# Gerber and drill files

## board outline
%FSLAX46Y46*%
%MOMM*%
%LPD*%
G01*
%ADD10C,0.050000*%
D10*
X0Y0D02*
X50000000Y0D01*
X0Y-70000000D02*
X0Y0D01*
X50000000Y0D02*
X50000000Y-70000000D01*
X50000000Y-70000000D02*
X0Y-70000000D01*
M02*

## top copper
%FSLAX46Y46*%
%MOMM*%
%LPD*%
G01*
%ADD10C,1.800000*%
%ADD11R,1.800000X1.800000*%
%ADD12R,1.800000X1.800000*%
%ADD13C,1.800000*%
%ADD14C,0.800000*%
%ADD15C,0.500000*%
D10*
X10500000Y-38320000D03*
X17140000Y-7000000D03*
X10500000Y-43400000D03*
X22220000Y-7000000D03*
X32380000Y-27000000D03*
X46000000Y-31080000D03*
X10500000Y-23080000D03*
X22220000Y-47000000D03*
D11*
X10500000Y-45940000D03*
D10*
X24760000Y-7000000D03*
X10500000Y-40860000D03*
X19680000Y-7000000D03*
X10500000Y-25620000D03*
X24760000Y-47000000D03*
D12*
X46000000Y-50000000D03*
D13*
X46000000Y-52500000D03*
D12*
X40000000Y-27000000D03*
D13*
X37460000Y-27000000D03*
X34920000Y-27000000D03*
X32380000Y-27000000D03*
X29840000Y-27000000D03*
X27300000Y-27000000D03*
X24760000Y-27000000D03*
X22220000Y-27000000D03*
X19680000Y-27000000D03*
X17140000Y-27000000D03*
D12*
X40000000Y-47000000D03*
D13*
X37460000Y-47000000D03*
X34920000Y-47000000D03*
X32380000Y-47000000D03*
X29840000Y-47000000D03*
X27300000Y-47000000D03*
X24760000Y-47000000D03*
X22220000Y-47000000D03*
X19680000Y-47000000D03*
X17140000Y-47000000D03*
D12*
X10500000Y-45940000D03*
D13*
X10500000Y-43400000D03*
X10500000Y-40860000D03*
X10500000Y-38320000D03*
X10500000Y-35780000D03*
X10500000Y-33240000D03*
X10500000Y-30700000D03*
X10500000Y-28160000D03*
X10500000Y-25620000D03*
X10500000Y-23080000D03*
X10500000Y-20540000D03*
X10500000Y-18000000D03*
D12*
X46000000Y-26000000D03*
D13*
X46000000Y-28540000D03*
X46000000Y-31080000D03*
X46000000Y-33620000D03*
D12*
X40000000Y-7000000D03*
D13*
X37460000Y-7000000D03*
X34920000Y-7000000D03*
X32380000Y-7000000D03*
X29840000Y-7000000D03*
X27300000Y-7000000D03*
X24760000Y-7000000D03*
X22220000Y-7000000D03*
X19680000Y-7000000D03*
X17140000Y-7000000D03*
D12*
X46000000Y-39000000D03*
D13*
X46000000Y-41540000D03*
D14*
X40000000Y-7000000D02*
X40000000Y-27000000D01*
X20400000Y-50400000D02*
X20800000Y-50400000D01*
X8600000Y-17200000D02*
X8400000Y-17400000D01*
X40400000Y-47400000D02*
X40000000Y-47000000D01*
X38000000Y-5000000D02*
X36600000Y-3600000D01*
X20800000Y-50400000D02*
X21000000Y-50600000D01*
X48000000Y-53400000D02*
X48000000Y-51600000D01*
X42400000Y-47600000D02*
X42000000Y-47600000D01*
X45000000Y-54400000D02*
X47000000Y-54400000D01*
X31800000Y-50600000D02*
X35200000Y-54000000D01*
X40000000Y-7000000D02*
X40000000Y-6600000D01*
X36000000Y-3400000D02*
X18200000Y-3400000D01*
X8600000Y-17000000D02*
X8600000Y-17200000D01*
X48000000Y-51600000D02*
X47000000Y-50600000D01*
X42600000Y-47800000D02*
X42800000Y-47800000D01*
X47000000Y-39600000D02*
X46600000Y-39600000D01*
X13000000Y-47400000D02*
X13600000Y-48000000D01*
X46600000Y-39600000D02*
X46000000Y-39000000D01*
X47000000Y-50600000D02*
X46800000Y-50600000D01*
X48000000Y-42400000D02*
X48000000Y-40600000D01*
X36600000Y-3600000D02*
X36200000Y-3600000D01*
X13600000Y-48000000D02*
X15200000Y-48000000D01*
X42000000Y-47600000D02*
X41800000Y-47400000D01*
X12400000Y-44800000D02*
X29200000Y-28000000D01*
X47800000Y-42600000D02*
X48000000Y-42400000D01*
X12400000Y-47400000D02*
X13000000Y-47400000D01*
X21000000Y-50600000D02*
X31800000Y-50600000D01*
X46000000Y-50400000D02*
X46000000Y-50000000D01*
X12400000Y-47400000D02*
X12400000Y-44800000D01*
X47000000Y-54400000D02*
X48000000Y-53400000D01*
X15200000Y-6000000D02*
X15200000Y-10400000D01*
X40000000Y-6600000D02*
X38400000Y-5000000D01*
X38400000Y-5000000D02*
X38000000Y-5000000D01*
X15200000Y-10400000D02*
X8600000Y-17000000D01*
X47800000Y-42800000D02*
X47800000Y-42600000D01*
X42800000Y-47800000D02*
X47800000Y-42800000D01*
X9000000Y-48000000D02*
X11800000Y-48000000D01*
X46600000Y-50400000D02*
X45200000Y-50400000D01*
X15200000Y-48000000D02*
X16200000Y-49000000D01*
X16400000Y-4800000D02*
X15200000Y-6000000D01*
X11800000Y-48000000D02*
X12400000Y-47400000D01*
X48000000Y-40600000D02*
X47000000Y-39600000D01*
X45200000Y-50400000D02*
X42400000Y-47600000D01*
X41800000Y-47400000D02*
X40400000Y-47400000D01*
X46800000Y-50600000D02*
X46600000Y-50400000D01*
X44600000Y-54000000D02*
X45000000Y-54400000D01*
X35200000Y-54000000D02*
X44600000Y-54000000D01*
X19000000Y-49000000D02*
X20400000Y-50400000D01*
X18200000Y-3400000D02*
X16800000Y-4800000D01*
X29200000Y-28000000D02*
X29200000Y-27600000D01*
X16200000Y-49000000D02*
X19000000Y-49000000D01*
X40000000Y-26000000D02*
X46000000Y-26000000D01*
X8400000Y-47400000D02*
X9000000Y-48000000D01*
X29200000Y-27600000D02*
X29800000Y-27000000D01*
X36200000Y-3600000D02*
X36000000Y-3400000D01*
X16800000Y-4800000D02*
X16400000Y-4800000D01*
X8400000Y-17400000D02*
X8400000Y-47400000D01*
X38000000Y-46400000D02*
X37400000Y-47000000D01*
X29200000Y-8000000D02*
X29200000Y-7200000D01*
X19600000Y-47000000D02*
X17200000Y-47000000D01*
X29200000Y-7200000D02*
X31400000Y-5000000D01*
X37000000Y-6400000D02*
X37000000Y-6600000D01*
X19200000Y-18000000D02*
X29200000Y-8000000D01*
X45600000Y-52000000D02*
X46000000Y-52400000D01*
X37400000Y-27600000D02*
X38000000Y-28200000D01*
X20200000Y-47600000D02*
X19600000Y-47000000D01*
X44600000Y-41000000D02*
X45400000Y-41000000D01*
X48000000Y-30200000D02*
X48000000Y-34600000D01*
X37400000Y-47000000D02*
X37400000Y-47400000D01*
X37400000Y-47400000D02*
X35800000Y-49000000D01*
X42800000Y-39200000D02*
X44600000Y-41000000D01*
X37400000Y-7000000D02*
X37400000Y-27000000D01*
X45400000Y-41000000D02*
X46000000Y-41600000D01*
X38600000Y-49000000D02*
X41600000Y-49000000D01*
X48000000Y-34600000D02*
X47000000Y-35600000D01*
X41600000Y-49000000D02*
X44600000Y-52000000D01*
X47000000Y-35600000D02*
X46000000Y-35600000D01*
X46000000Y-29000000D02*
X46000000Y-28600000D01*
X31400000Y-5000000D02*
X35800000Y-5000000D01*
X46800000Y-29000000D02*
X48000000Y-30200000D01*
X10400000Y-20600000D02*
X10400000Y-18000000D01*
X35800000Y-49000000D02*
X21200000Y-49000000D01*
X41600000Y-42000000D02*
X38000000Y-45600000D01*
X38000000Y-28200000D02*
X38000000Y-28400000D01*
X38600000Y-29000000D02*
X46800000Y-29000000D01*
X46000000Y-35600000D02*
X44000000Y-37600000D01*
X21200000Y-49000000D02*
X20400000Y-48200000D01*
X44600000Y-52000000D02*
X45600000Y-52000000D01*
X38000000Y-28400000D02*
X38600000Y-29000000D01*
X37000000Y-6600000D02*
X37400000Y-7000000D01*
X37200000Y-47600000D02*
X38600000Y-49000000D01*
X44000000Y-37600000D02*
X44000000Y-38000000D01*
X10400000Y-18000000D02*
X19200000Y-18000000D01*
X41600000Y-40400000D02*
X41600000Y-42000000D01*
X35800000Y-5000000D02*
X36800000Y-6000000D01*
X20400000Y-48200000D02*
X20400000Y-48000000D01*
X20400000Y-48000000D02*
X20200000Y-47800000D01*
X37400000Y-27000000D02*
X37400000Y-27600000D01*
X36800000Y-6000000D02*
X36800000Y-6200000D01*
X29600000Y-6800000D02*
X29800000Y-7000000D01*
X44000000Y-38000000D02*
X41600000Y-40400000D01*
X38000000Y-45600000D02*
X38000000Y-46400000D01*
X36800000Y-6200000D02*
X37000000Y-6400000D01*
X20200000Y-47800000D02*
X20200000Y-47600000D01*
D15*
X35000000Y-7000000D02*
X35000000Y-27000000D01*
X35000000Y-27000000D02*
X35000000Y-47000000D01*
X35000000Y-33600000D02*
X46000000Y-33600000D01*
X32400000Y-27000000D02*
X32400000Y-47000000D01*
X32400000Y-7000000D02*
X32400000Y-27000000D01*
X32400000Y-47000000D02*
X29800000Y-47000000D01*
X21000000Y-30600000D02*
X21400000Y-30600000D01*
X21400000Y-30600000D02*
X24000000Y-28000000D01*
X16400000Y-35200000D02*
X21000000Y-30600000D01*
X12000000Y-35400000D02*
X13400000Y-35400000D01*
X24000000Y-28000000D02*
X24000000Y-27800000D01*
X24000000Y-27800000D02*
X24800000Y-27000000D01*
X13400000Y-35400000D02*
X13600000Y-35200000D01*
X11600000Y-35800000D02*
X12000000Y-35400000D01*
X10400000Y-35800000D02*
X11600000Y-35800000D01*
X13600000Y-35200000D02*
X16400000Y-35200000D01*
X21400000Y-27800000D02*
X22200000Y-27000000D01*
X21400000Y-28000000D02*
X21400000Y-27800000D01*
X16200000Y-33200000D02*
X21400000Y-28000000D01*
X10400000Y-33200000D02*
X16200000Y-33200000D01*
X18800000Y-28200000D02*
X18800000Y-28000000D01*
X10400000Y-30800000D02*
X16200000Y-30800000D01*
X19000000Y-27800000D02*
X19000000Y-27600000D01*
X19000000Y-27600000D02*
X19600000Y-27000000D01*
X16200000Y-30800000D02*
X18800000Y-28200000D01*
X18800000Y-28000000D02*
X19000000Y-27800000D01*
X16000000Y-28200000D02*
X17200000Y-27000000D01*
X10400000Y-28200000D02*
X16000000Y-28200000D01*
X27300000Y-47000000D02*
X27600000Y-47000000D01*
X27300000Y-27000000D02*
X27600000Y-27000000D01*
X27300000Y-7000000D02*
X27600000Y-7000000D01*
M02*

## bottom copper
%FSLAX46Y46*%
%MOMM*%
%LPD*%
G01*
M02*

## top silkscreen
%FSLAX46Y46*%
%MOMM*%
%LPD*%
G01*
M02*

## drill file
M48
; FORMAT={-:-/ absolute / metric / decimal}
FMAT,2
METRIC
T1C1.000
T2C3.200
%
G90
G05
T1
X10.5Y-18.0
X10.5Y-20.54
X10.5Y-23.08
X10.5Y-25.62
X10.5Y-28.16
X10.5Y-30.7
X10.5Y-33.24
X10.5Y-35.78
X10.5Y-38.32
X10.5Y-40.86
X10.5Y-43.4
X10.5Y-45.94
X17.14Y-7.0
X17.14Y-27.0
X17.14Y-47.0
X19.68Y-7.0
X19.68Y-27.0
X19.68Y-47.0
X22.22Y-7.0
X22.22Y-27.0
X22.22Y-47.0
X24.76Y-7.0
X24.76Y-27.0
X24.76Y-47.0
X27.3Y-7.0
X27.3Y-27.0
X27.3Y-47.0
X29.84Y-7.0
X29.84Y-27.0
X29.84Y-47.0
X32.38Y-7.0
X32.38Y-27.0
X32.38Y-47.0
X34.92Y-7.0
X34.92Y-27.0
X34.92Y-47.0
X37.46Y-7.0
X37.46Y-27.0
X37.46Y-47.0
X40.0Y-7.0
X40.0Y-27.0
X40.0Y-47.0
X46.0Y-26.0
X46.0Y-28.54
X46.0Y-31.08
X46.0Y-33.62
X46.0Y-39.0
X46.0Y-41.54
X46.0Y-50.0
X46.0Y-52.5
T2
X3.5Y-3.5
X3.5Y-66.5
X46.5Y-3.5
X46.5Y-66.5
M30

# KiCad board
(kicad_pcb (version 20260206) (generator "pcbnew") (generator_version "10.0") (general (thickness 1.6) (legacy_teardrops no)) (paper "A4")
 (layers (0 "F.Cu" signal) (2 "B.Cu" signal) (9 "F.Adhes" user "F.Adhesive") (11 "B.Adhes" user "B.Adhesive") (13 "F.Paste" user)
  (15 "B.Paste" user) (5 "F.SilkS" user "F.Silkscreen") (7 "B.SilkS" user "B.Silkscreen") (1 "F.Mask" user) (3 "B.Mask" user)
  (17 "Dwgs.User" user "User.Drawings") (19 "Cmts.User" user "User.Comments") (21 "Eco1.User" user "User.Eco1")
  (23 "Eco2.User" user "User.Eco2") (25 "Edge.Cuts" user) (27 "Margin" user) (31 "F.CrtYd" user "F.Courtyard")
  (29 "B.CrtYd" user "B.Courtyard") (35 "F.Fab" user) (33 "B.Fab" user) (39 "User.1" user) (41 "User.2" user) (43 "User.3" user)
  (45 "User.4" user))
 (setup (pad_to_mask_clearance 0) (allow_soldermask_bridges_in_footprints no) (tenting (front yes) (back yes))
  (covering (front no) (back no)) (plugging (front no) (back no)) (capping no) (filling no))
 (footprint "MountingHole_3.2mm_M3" (layer "F.Cu") (at 3.5 3.5)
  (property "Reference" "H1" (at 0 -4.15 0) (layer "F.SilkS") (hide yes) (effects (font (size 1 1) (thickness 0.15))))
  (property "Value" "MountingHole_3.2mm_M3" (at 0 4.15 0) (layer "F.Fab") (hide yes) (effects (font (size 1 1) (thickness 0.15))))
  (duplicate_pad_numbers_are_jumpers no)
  (pad "" np_thru_hole circle (at 0 0) (size 3.2 3.2) (drill 3.2) (layers "*.Cu" "*.Mask")))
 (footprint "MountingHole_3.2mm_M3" (layer "F.Cu") (at 46.5 66.5)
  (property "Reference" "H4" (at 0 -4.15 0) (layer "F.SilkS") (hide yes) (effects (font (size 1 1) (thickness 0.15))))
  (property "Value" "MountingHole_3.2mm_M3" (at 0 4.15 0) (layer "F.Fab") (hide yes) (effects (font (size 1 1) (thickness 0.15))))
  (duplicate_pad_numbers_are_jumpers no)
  (pad "" np_thru_hole circle (at 0 0) (size 3.2 3.2) (drill 3.2) (layers "*.Cu" "*.Mask")))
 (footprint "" (layer "F.Cu") (at 0 0)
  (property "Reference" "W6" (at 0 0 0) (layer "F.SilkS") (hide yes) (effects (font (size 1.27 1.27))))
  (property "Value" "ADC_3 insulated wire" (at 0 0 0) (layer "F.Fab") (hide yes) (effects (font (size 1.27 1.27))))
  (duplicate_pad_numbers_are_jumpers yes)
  (pad "1" smd circle (at 10.5 38.32) (size 1.8 1.8) (layers "F.Cu") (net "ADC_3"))
  (pad "1" smd circle (at 17.14 7) (size 1.8 1.8) (layers "F.Cu") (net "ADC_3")))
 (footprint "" (layer "F.Cu") (at 0 0)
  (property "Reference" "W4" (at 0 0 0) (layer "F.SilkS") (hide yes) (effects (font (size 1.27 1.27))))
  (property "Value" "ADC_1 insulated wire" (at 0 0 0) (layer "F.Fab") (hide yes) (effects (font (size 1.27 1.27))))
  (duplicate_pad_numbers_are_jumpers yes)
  (pad "1" smd circle (at 10.5 43.4) (size 1.8 1.8) (layers "F.Cu") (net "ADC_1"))
  (pad "1" smd circle (at 22.22 7) (size 1.8 1.8) (layers "F.Cu") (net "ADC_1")))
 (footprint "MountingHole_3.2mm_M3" (layer "F.Cu") (at 3.5 66.5)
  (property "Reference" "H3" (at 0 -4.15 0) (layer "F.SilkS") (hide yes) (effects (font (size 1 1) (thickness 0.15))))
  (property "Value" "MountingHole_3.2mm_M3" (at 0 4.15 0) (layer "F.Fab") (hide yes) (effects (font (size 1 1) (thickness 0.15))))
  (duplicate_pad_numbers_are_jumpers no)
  (pad "" np_thru_hole circle (at 0 0) (size 3.2 3.2) (drill 3.2) (layers "*.Cu" "*.Mask")))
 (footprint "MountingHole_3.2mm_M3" (layer "F.Cu") (at 46.5 3.5)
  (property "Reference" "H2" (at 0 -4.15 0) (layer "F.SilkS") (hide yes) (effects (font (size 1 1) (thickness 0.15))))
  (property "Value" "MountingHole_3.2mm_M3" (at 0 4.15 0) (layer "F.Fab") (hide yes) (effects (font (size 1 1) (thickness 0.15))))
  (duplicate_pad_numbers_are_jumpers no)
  (pad "" np_thru_hole circle (at 0 0) (size 3.2 3.2) (drill 3.2) (layers "*.Cu" "*.Mask")))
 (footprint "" (layer "F.Cu") (at 0 0)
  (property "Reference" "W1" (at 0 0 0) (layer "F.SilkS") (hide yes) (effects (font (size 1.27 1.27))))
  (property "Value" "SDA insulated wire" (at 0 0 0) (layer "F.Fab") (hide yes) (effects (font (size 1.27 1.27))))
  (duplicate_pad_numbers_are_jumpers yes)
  (pad "1" smd circle (at 32.38 27) (size 1.8 1.8) (layers "F.Cu") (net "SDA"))
  (pad "1" smd circle (at 46 31.08) (size 1.8 1.8) (layers "F.Cu") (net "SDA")))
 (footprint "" (layer "F.Cu") (at 0 0)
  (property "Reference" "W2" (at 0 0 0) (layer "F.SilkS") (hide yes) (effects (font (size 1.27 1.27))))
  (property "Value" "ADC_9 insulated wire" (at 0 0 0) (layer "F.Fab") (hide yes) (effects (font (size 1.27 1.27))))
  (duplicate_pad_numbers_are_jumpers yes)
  (pad "1" smd circle (at 10.5 23.08) (size 1.8 1.8) (layers "F.Cu") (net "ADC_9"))
  (pad "1" smd circle (at 22.22 47) (size 1.8 1.8) (layers "F.Cu") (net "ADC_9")))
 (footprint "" (layer "F.Cu") (at 0 0)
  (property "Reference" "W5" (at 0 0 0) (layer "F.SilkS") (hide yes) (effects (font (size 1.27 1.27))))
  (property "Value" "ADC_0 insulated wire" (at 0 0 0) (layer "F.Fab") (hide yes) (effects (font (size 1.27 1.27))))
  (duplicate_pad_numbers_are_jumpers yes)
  (pad "1" smd rect (at 10.5 45.94) (size 1.8 1.8) (layers "F.Cu") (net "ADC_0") (thermal_bridge_angle 45))
  (pad "1" smd circle (at 24.76 7) (size 1.8 1.8) (layers "F.Cu") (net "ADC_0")))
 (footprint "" (layer "F.Cu") (at 0 0)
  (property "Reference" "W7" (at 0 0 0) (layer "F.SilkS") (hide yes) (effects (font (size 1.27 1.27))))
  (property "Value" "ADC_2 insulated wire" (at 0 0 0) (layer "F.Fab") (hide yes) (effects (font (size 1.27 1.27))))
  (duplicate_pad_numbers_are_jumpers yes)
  (pad "1" smd circle (at 10.5 40.86) (size 1.8 1.8) (layers "F.Cu") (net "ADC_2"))
  (pad "1" smd circle (at 19.68 7) (size 1.8 1.8) (layers "F.Cu") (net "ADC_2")))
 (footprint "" (layer "F.Cu") (at 0 0)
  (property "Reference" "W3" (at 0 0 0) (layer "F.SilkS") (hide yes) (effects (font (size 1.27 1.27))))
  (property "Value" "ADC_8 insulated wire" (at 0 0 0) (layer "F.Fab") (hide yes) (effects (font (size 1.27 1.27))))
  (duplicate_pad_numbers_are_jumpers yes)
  (pad "1" smd circle (at 10.5 25.62) (size 1.8 1.8) (layers "F.Cu") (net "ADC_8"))
  (pad "1" smd circle (at 24.76 47) (size 1.8 1.8) (layers "F.Cu") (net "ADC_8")))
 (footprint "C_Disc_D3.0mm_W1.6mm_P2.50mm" (layer "B.Cu") (at 46 50 -90)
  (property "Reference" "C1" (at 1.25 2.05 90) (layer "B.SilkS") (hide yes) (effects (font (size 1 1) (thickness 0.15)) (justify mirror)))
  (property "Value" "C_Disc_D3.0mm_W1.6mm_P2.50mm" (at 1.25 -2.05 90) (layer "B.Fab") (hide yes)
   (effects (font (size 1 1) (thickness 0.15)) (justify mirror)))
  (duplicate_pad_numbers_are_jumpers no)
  (pad "1" thru_hole rect (at 0 0 270) (size 1.8 1.8) (drill 1) (layers "*.Mask" "F.Cu") (remove_unused_layers yes) (keep_end_layers no)
   (zone_layer_connections) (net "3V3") (thermal_bridge_angle 45))
  (pad "2" thru_hole circle (at 2.5 0 270) (size 1.8 1.8) (drill 1) (layers "*.Mask" "F.Cu") (remove_unused_layers yes) (keep_end_layers no)
   (zone_layer_connections) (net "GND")))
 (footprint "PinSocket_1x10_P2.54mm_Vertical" (layer "B.Cu") (at 40 27 90)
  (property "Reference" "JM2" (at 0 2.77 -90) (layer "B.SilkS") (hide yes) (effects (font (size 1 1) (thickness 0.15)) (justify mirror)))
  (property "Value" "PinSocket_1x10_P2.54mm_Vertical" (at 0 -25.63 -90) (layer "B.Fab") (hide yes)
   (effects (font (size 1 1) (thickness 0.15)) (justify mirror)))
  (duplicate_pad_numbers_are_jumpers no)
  (pad "1" thru_hole rect (at 0 0 90) (size 1.8 1.8) (drill 1) (layers "*.Mask" "F.Cu") (remove_unused_layers yes) (keep_end_layers no)
   (zone_layer_connections) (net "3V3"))
  (pad "2" thru_hole circle (at 0 -2.54 90) (size 1.8 1.8) (drill 1) (layers "*.Mask" "F.Cu") (remove_unused_layers yes)
   (keep_end_layers no) (zone_layer_connections) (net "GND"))
  (pad "3" thru_hole circle (at 0 -5.08 90) (size 1.8 1.8) (drill 1) (layers "*.Mask" "F.Cu") (remove_unused_layers yes)
   (keep_end_layers no) (zone_layer_connections) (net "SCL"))
  (pad "4" thru_hole circle (at 0 -7.62 90) (size 1.8 1.8) (drill 1) (layers "*.Mask" "F.Cu") (remove_unused_layers yes)
   (keep_end_layers no) (zone_layer_connections) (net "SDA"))
  (pad "5" thru_hole circle (at 0 -10.16 90) (size 1.8 1.8) (drill 1) (layers "*.Mask" "F.Cu") (remove_unused_layers yes)
   (keep_end_layers no) (zone_layer_connections) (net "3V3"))
  (pad "6" thru_hole circle (at 0 -12.7 90) (size 1.8 1.8) (drill 1) (layers "*.Mask" "F.Cu") (remove_unused_layers yes)
   (keep_end_layers no) (zone_layer_connections) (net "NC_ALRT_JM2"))
  (pad "7" thru_hole circle (at 0 -15.24 90) (size 1.8 1.8) (drill 1) (layers "*.Mask" "F.Cu") (remove_unused_layers yes)
   (keep_end_layers no) (zone_layer_connections) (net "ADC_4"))
  (pad "8" thru_hole circle (at 0 -17.78 90) (size 1.8 1.8) (drill 1) (layers "*.Mask" "F.Cu") (remove_unused_layers yes)
   (keep_end_layers no) (zone_layer_connections) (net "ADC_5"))
  (pad "9" thru_hole circle (at 0 -20.32 90) (size 1.8 1.8) (drill 1) (layers "*.Mask" "F.Cu") (remove_unused_layers yes)
   (keep_end_layers no) (zone_layer_connections) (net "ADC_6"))
  (pad "10" thru_hole circle (at 0 -22.86 90) (size 1.8 1.8) (drill 1) (layers "*.Mask" "F.Cu") (remove_unused_layers yes)
   (keep_end_layers no) (zone_layer_connections) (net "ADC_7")))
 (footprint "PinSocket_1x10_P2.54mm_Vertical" (layer "B.Cu") (at 40 47 90)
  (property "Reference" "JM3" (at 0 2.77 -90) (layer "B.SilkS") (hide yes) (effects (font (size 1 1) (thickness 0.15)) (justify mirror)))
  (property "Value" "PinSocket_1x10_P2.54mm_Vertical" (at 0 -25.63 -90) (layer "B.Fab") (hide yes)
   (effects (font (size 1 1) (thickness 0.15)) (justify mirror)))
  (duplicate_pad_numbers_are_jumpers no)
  (pad "1" thru_hole rect (at 0 0 90) (size 1.8 1.8) (drill 1) (layers "*.Mask" "F.Cu") (remove_unused_layers yes) (keep_end_layers no)
   (zone_layer_connections) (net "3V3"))
  (pad "2" thru_hole circle (at 0 -2.54 90) (size 1.8 1.8) (drill 1) (layers "*.Mask" "F.Cu") (remove_unused_layers yes)
   (keep_end_layers no) (zone_layer_connections) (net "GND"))
  (pad "3" thru_hole circle (at 0 -5.08 90) (size 1.8 1.8) (drill 1) (layers "*.Mask" "F.Cu") (remove_unused_layers yes)
   (keep_end_layers no) (zone_layer_connections) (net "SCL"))
  (pad "4" thru_hole circle (at 0 -7.62 90) (size 1.8 1.8) (drill 1) (layers "*.Mask" "F.Cu") (remove_unused_layers yes)
   (keep_end_layers no) (zone_layer_connections) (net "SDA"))
  (pad "5" thru_hole circle (at 0 -10.16 90) (size 1.8 1.8) (drill 1) (layers "*.Mask" "F.Cu") (remove_unused_layers yes)
   (keep_end_layers no) (zone_layer_connections) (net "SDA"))
  (pad "6" thru_hole circle (at 0 -12.7 90) (size 1.8 1.8) (drill 1) (layers "*.Mask" "F.Cu") (remove_unused_layers yes)
   (keep_end_layers no) (zone_layer_connections) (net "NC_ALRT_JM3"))
  (pad "7" thru_hole circle (at 0 -15.24 90) (size 1.8 1.8) (drill 1) (layers "*.Mask" "F.Cu") (remove_unused_layers yes)
   (keep_end_layers no) (zone_layer_connections) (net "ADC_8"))
  (pad "8" thru_hole circle (at 0 -17.78 90) (size 1.8 1.8) (drill 1) (layers "*.Mask" "F.Cu") (remove_unused_layers yes)
   (keep_end_layers no) (zone_layer_connections) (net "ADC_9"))
  (pad "9" thru_hole circle (at 0 -20.32 90) (size 1.8 1.8) (drill 1) (layers "*.Mask" "F.Cu") (remove_unused_layers yes)
   (keep_end_layers no) (zone_layer_connections) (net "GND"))
  (pad "10" thru_hole circle (at 0 -22.86 90) (size 1.8 1.8) (drill 1) (layers "*.Mask" "F.Cu") (remove_unused_layers yes)
   (keep_end_layers no) (zone_layer_connections) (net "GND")))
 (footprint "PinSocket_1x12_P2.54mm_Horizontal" (layer "B.Cu") (at 10.5 45.94)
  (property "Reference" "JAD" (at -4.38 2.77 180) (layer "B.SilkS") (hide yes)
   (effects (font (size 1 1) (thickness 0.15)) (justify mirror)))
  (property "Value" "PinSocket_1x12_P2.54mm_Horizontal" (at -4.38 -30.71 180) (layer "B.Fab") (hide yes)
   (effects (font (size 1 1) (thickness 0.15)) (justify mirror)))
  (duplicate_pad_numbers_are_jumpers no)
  (pad "1" thru_hole rect (at 0 0) (size 1.8 1.8) (drill 1) (layers "*.Mask" "F.Cu") (remove_unused_layers yes) (keep_end_layers no)
   (zone_layer_connections) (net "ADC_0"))
  (pad "2" thru_hole circle (at 0 -2.54) (size 1.8 1.8) (drill 1) (layers "*.Mask" "F.Cu") (remove_unused_layers yes) (keep_end_layers no)
   (zone_layer_connections) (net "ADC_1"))
  (pad "3" thru_hole circle (at 0 -5.08) (size 1.8 1.8) (drill 1) (layers "*.Mask" "F.Cu") (remove_unused_layers yes) (keep_end_layers no)
   (zone_layer_connections) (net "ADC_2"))
  (pad "4" thru_hole circle (at 0 -7.62) (size 1.8 1.8) (drill 1) (layers "*.Mask" "F.Cu") (remove_unused_layers yes) (keep_end_layers no)
   (zone_layer_connections) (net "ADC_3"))
  (pad "5" thru_hole circle (at 0 -10.16) (size 1.8 1.8) (drill 1) (layers "*.Mask" "F.Cu") (remove_unused_layers yes) (keep_end_layers no)
   (zone_layer_connections) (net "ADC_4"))
  (pad "6" thru_hole circle (at 0 -12.7) (size 1.8 1.8) (drill 1) (layers "*.Mask" "F.Cu") (remove_unused_layers yes) (keep_end_layers no)
   (zone_layer_connections) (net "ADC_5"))
  (pad "7" thru_hole circle (at 0 -15.24) (size 1.8 1.8) (drill 1) (layers "*.Mask" "F.Cu") (remove_unused_layers yes) (keep_end_layers no)
   (zone_layer_connections) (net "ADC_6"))
  (pad "8" thru_hole circle (at 0 -17.78) (size 1.8 1.8) (drill 1) (layers "*.Mask" "F.Cu") (remove_unused_layers yes) (keep_end_layers no)
   (zone_layer_connections) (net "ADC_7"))
  (pad "9" thru_hole circle (at 0 -20.32) (size 1.8 1.8) (drill 1) (layers "*.Mask" "F.Cu") (remove_unused_layers yes) (keep_end_layers no)
   (zone_layer_connections) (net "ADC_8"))
  (pad "10" thru_hole circle (at 0 -22.86) (size 1.8 1.8) (drill 1) (layers "*.Mask" "F.Cu") (remove_unused_layers yes) (keep_end_layers no)
   (zone_layer_connections) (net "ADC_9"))
  (pad "11" thru_hole circle (at 0 -25.4) (size 1.8 1.8) (drill 1) (layers "*.Mask" "F.Cu") (remove_unused_layers yes) (keep_end_layers no)
   (zone_layer_connections) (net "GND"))
  (pad "12" thru_hole circle (at 0 -27.94) (size 1.8 1.8) (drill 1) (layers "*.Mask" "F.Cu") (remove_unused_layers yes) (keep_end_layers no)
   (zone_layer_connections) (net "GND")))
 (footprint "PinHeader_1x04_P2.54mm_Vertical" (layer "B.Cu") (at 46 26 180)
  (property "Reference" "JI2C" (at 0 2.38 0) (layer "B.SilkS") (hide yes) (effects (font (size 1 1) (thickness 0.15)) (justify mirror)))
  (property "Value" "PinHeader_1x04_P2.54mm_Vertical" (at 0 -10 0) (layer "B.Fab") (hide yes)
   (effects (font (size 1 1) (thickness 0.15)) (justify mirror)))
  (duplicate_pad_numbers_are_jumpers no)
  (pad "1" thru_hole rect (at 0 0 180) (size 1.8 1.8) (drill 1) (layers "*.Mask" "F.Cu") (remove_unused_layers yes) (keep_end_layers no)
   (zone_layer_connections) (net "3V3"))
  (pad "2" thru_hole circle (at 0 -2.54 180) (size 1.8 1.8) (drill 1) (layers "*.Mask" "F.Cu") (remove_unused_layers yes)
   (keep_end_layers no) (zone_layer_connections) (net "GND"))
  (pad "3" thru_hole circle (at 0 -5.08 180) (size 1.8 1.8) (drill 1) (layers "*.Mask" "F.Cu") (remove_unused_layers yes)
   (keep_end_layers no) (zone_layer_connections) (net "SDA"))
  (pad "4" thru_hole circle (at 0 -7.62 180) (size 1.8 1.8) (drill 1) (layers "*.Mask" "F.Cu") (remove_unused_layers yes)
   (keep_end_layers no) (zone_layer_connections) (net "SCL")))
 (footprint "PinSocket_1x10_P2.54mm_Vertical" (layer "B.Cu") (at 40 7 90)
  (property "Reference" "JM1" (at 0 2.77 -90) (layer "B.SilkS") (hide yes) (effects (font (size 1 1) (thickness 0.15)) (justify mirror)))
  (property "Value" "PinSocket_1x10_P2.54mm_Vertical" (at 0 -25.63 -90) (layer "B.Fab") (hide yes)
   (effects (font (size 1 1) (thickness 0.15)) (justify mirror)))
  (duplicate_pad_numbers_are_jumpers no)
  (pad "1" thru_hole rect (at 0 0 90) (size 1.8 1.8) (drill 1) (layers "*.Mask" "F.Cu") (remove_unused_layers yes) (keep_end_layers no)
   (zone_layer_connections) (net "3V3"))
  (pad "2" thru_hole circle (at 0 -2.54 90) (size 1.8 1.8) (drill 1) (layers "*.Mask" "F.Cu") (remove_unused_layers yes)
   (keep_end_layers no) (zone_layer_connections) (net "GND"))
  (pad "3" thru_hole circle (at 0 -5.08 90) (size 1.8 1.8) (drill 1) (layers "*.Mask" "F.Cu") (remove_unused_layers yes)
   (keep_end_layers no) (zone_layer_connections) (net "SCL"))
  (pad "4" thru_hole circle (at 0 -7.62 90) (size 1.8 1.8) (drill 1) (layers "*.Mask" "F.Cu") (remove_unused_layers yes)
   (keep_end_layers no) (zone_layer_connections) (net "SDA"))
  (pad "5" thru_hole circle (at 0 -10.16 90) (size 1.8 1.8) (drill 1) (layers "*.Mask" "F.Cu") (remove_unused_layers yes)
   (keep_end_layers no) (zone_layer_connections) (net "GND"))
  (pad "6" thru_hole circle (at 0 -12.7 90) (size 1.8 1.8) (drill 1) (layers "*.Mask" "F.Cu") (remove_unused_layers yes)
   (keep_end_layers no) (zone_layer_connections) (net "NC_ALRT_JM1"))
  (pad "7" thru_hole circle (at 0 -15.24 90) (size 1.8 1.8) (drill 1) (layers "*.Mask" "F.Cu") (remove_unused_layers yes)
   (keep_end_layers no) (zone_layer_connections) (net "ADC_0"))
  (pad "8" thru_hole circle (at 0 -17.78 90) (size 1.8 1.8) (drill 1) (layers "*.Mask" "F.Cu") (remove_unused_layers yes)
   (keep_end_layers no) (zone_layer_connections) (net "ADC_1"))
  (pad "9" thru_hole circle (at 0 -20.32 90) (size 1.8 1.8) (drill 1) (layers "*.Mask" "F.Cu") (remove_unused_layers yes)
   (keep_end_layers no) (zone_layer_connections) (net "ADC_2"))
  (pad "10" thru_hole circle (at 0 -22.86 90) (size 1.8 1.8) (drill 1) (layers "*.Mask" "F.Cu") (remove_unused_layers yes)
   (keep_end_layers no) (zone_layer_connections) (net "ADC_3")))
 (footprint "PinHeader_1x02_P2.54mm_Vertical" (layer "B.Cu") (at 46 39 180)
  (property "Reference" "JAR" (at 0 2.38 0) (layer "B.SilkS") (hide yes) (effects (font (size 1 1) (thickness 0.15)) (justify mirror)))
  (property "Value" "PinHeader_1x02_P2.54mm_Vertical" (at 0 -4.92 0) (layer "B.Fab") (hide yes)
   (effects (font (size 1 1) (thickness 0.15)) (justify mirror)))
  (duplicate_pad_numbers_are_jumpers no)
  (pad "1" thru_hole rect (at 0 0 180) (size 1.8 1.8) (drill 1) (layers "*.Mask" "F.Cu") (remove_unused_layers yes) (keep_end_layers no)
   (zone_layer_connections) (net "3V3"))
  (pad "2" thru_hole circle (at 0 -2.54 180) (size 1.8 1.8) (drill 1) (layers "*.Mask" "F.Cu") (remove_unused_layers yes)
   (keep_end_layers no) (zone_layer_connections) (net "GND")))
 (gr_line (start 0 0) (end 50 0) (stroke (width 0.05) (type default)) (layer "Edge.Cuts"))
 (gr_line (start 0 70) (end 0 0) (stroke (width 0.05) (type default)) (layer "Edge.Cuts"))
 (gr_line (start 50 0) (end 50 70) (stroke (width 0.05) (type default)) (layer "Edge.Cuts"))
 (gr_line (start 50 70) (end 0 70) (stroke (width 0.05) (type default)) (layer "Edge.Cuts"))
 (segment (start 40 7) (end 40 27) (width 0.8) (layer "F.Cu") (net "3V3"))
 (segment (start 20.4 50.4) (end 20.8 50.4) (width 0.8) (layer "F.Cu") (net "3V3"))
 (segment (start 8.6 17.2) (end 8.4 17.4) (width 0.8) (layer "F.Cu") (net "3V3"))
 (segment (start 40.4 47.4) (end 40 47) (width 0.8) (layer "F.Cu") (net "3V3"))
 (segment (start 38 5) (end 36.6 3.6) (width 0.8) (layer "F.Cu") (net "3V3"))
 (segment (start 20.8 50.4) (end 21 50.6) (width 0.8) (layer "F.Cu") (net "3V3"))
 (segment (start 48 53.4) (end 48 51.6) (width 0.8) (layer "F.Cu") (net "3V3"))
 (segment (start 42.4 47.6) (end 42 47.6) (width 0.8) (layer "F.Cu") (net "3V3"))
 (segment (start 45 54.4) (end 47 54.4) (width 0.8) (layer "F.Cu") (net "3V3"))
 (segment (start 31.8 50.6) (end 35.2 54) (width 0.8) (layer "F.Cu") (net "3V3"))
 (segment (start 40 7) (end 40 6.6) (width 0.8) (layer "F.Cu") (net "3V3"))
 (segment (start 36 3.4) (end 18.2 3.4) (width 0.8) (layer "F.Cu") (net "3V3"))
 (segment (start 8.6 17) (end 8.6 17.2) (width 0.8) (layer "F.Cu") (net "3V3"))
 (segment (start 48 51.6) (end 47 50.6) (width 0.8) (layer "F.Cu") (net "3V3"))
 (segment (start 42.6 47.8) (end 42.8 47.8) (width 0.8) (layer "F.Cu") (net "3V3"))
 (segment (start 47 39.6) (end 46.6 39.6) (width 0.8) (layer "F.Cu") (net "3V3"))
 (segment (start 13 47.4) (end 13.6 48) (width 0.8) (layer "F.Cu") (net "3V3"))
 (segment (start 46.6 39.6) (end 46 39) (width 0.8) (layer "F.Cu") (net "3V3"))
 (segment (start 47 50.6) (end 46.8 50.6) (width 0.8) (layer "F.Cu") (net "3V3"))
 (segment (start 48 42.4) (end 48 40.6) (width 0.8) (layer "F.Cu") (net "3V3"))
 (segment (start 36.6 3.6) (end 36.2 3.6) (width 0.8) (layer "F.Cu") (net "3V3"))
 (segment (start 13.6 48) (end 15.2 48) (width 0.8) (layer "F.Cu") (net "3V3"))
 (segment (start 42 47.6) (end 41.8 47.4) (width 0.8) (layer "F.Cu") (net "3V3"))
 (segment (start 12.4 44.8) (end 29.2 28) (width 0.8) (layer "F.Cu") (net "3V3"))
 (segment (start 47.8 42.6) (end 48 42.4) (width 0.8) (layer "F.Cu") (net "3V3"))
 (segment (start 12.4 47.4) (end 13 47.4) (width 0.8) (layer "F.Cu") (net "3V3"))
 (segment (start 21 50.6) (end 31.8 50.6) (width 0.8) (layer "F.Cu") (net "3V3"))
 (segment (start 46 50.4) (end 46 50) (width 0.8) (layer "F.Cu") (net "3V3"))
 (segment (start 12.4 47.4) (end 12.4 44.8) (width 0.8) (layer "F.Cu") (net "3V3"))
 (segment (start 47 54.4) (end 48 53.4) (width 0.8) (layer "F.Cu") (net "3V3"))
 (segment (start 15.2 6) (end 15.2 10.4) (width 0.8) (layer "F.Cu") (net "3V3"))
 (segment (start 40 6.6) (end 38.4 5) (width 0.8) (layer "F.Cu") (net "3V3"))
 (segment (start 38.4 5) (end 38 5) (width 0.8) (layer "F.Cu") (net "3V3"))
 (segment (start 15.2 10.4) (end 8.6 17) (width 0.8) (layer "F.Cu") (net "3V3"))
 (segment (start 47.8 42.8) (end 47.8 42.6) (width 0.8) (layer "F.Cu") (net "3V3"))
 (segment (start 42.8 47.8) (end 47.8 42.8) (width 0.8) (layer "F.Cu") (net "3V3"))
 (segment (start 9 48) (end 11.8 48) (width 0.8) (layer "F.Cu") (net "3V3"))
 (segment (start 46.6 50.4) (end 45.2 50.4) (width 0.8) (layer "F.Cu") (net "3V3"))
 (segment (start 15.2 48) (end 16.2 49) (width 0.8) (layer "F.Cu") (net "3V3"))
 (segment (start 16.4 4.8) (end 15.2 6) (width 0.8) (layer "F.Cu") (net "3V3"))
 (segment (start 11.8 48) (end 12.4 47.4) (width 0.8) (layer "F.Cu") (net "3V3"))
 (segment (start 48 40.6) (end 47 39.6) (width 0.8) (layer "F.Cu") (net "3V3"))
 (segment (start 45.2 50.4) (end 42.4 47.6) (width 0.8) (layer "F.Cu") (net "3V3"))
 (segment (start 41.8 47.4) (end 40.4 47.4) (width 0.8) (layer "F.Cu") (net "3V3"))
 (segment (start 46.8 50.6) (end 46.6 50.4) (width 0.8) (layer "F.Cu") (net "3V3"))
 (segment (start 44.6 54) (end 45 54.4) (width 0.8) (layer "F.Cu") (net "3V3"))
 (segment (start 35.2 54) (end 44.6 54) (width 0.8) (layer "F.Cu") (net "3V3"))
 (segment (start 19 49) (end 20.4 50.4) (width 0.8) (layer "F.Cu") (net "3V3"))
 (segment (start 18.2 3.4) (end 16.8 4.8) (width 0.8) (layer "F.Cu") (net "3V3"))
 (segment (start 29.2 28) (end 29.2 27.6) (width 0.8) (layer "F.Cu") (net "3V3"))
 (segment (start 16.2 49) (end 19 49) (width 0.8) (layer "F.Cu") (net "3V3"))
 (segment (start 40 26) (end 46 26) (width 0.8) (layer "F.Cu") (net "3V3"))
 (segment (start 8.4 47.4) (end 9 48) (width 0.8) (layer "F.Cu") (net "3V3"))
 (segment (start 29.2 27.6) (end 29.8 27) (width 0.8) (layer "F.Cu") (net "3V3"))
 (segment (start 36.2 3.6) (end 36 3.4) (width 0.8) (layer "F.Cu") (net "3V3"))
 (segment (start 16.8 4.8) (end 16.4 4.8) (width 0.8) (layer "F.Cu") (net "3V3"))
 (segment (start 8.4 17.4) (end 8.4 47.4) (width 0.8) (layer "F.Cu") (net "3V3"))
 (segment (start 38 46.4) (end 37.4 47) (width 0.8) (layer "F.Cu") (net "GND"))
 (segment (start 29.2 8) (end 29.2 7.2) (width 0.8) (layer "F.Cu") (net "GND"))
 (segment (start 19.6 47) (end 17.2 47) (width 0.8) (layer "F.Cu") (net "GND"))
 (segment (start 29.2 7.2) (end 31.4 5) (width 0.8) (layer "F.Cu") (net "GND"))
 (segment (start 37 6.4) (end 37 6.6) (width 0.8) (layer "F.Cu") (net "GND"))
 (segment (start 19.2 18) (end 29.2 8) (width 0.8) (layer "F.Cu") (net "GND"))
 (segment (start 45.6 52) (end 46 52.4) (width 0.8) (layer "F.Cu") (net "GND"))
 (segment (start 37.4 27.6) (end 38 28.2) (width 0.8) (layer "F.Cu") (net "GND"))
 (segment (start 20.2 47.6) (end 19.6 47) (width 0.8) (layer "F.Cu") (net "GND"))
 (segment (start 44.6 41) (end 45.4 41) (width 0.8) (layer "F.Cu") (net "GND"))
 (segment (start 48 30.2) (end 48 34.6) (width 0.8) (layer "F.Cu") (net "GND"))
 (segment (start 37.4 47) (end 37.4 47.4) (width 0.8) (layer "F.Cu") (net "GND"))
 (segment (start 37.4 47.4) (end 35.8 49) (width 0.8) (layer "F.Cu") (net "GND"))
 (segment (start 42.8 39.2) (end 44.6 41) (width 0.8) (layer "F.Cu") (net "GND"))
 (segment (start 37.4 7) (end 37.4 27) (width 0.8) (layer "F.Cu") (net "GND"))
 (segment (start 45.4 41) (end 46 41.6) (width 0.8) (layer "F.Cu") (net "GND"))
 (segment (start 38.6 49) (end 41.6 49) (width 0.8) (layer "F.Cu") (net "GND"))
 (segment (start 48 34.6) (end 47 35.6) (width 0.8) (layer "F.Cu") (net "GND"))
 (segment (start 41.6 49) (end 44.6 52) (width 0.8) (layer "F.Cu") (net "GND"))
 (segment (start 47 35.6) (end 46 35.6) (width 0.8) (layer "F.Cu") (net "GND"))
 (segment (start 46 29) (end 46 28.6) (width 0.8) (layer "F.Cu") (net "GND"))
 (segment (start 31.4 5) (end 35.8 5) (width 0.8) (layer "F.Cu") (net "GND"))
 (segment (start 46.8 29) (end 48 30.2) (width 0.8) (layer "F.Cu") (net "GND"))
 (segment (start 10.4 20.6) (end 10.4 18) (width 0.8) (layer "F.Cu") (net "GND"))
 (segment (start 35.8 49) (end 21.2 49) (width 0.8) (layer "F.Cu") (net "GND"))
 (segment (start 41.6 42) (end 38 45.6) (width 0.8) (layer "F.Cu") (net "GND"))
 (segment (start 38 28.2) (end 38 28.4) (width 0.8) (layer "F.Cu") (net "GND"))
 (segment (start 38.6 29) (end 46.8 29) (width 0.8) (layer "F.Cu") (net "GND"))
 (segment (start 46 35.6) (end 44 37.6) (width 0.8) (layer "F.Cu") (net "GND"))
 (segment (start 21.2 49) (end 20.4 48.2) (width 0.8) (layer "F.Cu") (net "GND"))
 (segment (start 44.6 52) (end 45.6 52) (width 0.8) (layer "F.Cu") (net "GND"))
 (segment (start 38 28.4) (end 38.6 29) (width 0.8) (layer "F.Cu") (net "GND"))
 (segment (start 37 6.6) (end 37.4 7) (width 0.8) (layer "F.Cu") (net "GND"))
 (segment (start 37.2 47.6) (end 38.6 49) (width 0.8) (layer "F.Cu") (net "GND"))
 (segment (start 44 37.6) (end 44 38) (width 0.8) (layer "F.Cu") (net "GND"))
 (segment (start 10.4 18) (end 19.2 18) (width 0.8) (layer "F.Cu") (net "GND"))
 (segment (start 41.6 40.4) (end 41.6 42) (width 0.8) (layer "F.Cu") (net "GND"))
 (segment (start 35.8 5) (end 36.8 6) (width 0.8) (layer "F.Cu") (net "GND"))
 (segment (start 20.4 48.2) (end 20.4 48) (width 0.8) (layer "F.Cu") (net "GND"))
 (segment (start 20.4 48) (end 20.2 47.8) (width 0.8) (layer "F.Cu") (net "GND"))
 (segment (start 37.4 27) (end 37.4 27.6) (width 0.8) (layer "F.Cu") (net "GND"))
 (segment (start 36.8 6) (end 36.8 6.2) (width 0.8) (layer "F.Cu") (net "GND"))
 (segment (start 29.6 6.8) (end 29.8 7) (width 0.8) (layer "F.Cu") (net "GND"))
 (segment (start 44 38) (end 41.6 40.4) (width 0.8) (layer "F.Cu") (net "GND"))
 (segment (start 38 45.6) (end 38 46.4) (width 0.8) (layer "F.Cu") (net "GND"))
 (segment (start 36.8 6.2) (end 37 6.4) (width 0.8) (layer "F.Cu") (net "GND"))
 (segment (start 20.2 47.8) (end 20.2 47.6) (width 0.8) (layer "F.Cu") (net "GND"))
 (segment (start 35 7) (end 35 27) (width 0.5) (layer "F.Cu") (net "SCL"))
 (segment (start 35 27) (end 35 47) (width 0.5) (layer "F.Cu") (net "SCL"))
 (segment (start 35 33.6) (end 46 33.6) (width 0.5) (layer "F.Cu") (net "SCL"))
 (segment (start 32.4 27) (end 32.4 47) (width 0.5) (layer "F.Cu") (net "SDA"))
 (segment (start 32.4 7) (end 32.4 27) (width 0.5) (layer "F.Cu") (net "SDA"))
 (segment (start 32.4 47) (end 29.8 47) (width 0.5) (layer "F.Cu") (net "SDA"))
 (segment (start 21 30.6) (end 21.4 30.6) (width 0.5) (layer "F.Cu") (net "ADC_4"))
 (segment (start 21.4 30.6) (end 24 28) (width 0.5) (layer "F.Cu") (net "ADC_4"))
 (segment (start 16.4 35.2) (end 21 30.6) (width 0.5) (layer "F.Cu") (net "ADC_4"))
 (segment (start 12 35.4) (end 13.4 35.4) (width 0.5) (layer "F.Cu") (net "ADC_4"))
 (segment (start 24 28) (end 24 27.8) (width 0.5) (layer "F.Cu") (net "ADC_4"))
 (segment (start 24 27.8) (end 24.8 27) (width 0.5) (layer "F.Cu") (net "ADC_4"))
 (segment (start 13.4 35.4) (end 13.6 35.2) (width 0.5) (layer "F.Cu") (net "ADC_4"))
 (segment (start 11.6 35.8) (end 12 35.4) (width 0.5) (layer "F.Cu") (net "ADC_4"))
 (segment (start 10.4 35.8) (end 11.6 35.8) (width 0.5) (layer "F.Cu") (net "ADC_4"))
 (segment (start 13.6 35.2) (end 16.4 35.2) (width 0.5) (layer "F.Cu") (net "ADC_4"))
 (segment (start 21.4 27.8) (end 22.2 27) (width 0.5) (layer "F.Cu") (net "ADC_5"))
 (segment (start 21.4 28) (end 21.4 27.8) (width 0.5) (layer "F.Cu") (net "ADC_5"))
 (segment (start 16.2 33.2) (end 21.4 28) (width 0.5) (layer "F.Cu") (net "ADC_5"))
 (segment (start 10.4 33.2) (end 16.2 33.2) (width 0.5) (layer "F.Cu") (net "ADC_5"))
 (segment (start 18.8 28.2) (end 18.8 28) (width 0.5) (layer "F.Cu") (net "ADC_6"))
 (segment (start 10.4 30.8) (end 16.2 30.8) (width 0.5) (layer "F.Cu") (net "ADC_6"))
 (segment (start 19 27.8) (end 19 27.6) (width 0.5) (layer "F.Cu") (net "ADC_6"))
 (segment (start 19 27.6) (end 19.6 27) (width 0.5) (layer "F.Cu") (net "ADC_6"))
 (segment (start 16.2 30.8) (end 18.8 28.2) (width 0.5) (layer "F.Cu") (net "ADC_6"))
 (segment (start 18.8 28) (end 19 27.8) (width 0.5) (layer "F.Cu") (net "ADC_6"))
 (segment (start 16 28.2) (end 17.2 27) (width 0.5) (layer "F.Cu") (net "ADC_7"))
 (segment (start 10.4 28.2) (end 16 28.2) (width 0.5) (layer "F.Cu") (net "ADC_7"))
 (segment (start 27.3 47) (end 27.6 47) (width 0.5) (layer "F.Cu") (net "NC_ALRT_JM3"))
 (segment (start 27.3 27) (end 27.6 27) (width 0.5) (layer "F.Cu") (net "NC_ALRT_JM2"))
 (segment (start 27.3 7) (end 27.6 7) (width 0.5) (layer "F.Cu") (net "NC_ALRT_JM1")))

